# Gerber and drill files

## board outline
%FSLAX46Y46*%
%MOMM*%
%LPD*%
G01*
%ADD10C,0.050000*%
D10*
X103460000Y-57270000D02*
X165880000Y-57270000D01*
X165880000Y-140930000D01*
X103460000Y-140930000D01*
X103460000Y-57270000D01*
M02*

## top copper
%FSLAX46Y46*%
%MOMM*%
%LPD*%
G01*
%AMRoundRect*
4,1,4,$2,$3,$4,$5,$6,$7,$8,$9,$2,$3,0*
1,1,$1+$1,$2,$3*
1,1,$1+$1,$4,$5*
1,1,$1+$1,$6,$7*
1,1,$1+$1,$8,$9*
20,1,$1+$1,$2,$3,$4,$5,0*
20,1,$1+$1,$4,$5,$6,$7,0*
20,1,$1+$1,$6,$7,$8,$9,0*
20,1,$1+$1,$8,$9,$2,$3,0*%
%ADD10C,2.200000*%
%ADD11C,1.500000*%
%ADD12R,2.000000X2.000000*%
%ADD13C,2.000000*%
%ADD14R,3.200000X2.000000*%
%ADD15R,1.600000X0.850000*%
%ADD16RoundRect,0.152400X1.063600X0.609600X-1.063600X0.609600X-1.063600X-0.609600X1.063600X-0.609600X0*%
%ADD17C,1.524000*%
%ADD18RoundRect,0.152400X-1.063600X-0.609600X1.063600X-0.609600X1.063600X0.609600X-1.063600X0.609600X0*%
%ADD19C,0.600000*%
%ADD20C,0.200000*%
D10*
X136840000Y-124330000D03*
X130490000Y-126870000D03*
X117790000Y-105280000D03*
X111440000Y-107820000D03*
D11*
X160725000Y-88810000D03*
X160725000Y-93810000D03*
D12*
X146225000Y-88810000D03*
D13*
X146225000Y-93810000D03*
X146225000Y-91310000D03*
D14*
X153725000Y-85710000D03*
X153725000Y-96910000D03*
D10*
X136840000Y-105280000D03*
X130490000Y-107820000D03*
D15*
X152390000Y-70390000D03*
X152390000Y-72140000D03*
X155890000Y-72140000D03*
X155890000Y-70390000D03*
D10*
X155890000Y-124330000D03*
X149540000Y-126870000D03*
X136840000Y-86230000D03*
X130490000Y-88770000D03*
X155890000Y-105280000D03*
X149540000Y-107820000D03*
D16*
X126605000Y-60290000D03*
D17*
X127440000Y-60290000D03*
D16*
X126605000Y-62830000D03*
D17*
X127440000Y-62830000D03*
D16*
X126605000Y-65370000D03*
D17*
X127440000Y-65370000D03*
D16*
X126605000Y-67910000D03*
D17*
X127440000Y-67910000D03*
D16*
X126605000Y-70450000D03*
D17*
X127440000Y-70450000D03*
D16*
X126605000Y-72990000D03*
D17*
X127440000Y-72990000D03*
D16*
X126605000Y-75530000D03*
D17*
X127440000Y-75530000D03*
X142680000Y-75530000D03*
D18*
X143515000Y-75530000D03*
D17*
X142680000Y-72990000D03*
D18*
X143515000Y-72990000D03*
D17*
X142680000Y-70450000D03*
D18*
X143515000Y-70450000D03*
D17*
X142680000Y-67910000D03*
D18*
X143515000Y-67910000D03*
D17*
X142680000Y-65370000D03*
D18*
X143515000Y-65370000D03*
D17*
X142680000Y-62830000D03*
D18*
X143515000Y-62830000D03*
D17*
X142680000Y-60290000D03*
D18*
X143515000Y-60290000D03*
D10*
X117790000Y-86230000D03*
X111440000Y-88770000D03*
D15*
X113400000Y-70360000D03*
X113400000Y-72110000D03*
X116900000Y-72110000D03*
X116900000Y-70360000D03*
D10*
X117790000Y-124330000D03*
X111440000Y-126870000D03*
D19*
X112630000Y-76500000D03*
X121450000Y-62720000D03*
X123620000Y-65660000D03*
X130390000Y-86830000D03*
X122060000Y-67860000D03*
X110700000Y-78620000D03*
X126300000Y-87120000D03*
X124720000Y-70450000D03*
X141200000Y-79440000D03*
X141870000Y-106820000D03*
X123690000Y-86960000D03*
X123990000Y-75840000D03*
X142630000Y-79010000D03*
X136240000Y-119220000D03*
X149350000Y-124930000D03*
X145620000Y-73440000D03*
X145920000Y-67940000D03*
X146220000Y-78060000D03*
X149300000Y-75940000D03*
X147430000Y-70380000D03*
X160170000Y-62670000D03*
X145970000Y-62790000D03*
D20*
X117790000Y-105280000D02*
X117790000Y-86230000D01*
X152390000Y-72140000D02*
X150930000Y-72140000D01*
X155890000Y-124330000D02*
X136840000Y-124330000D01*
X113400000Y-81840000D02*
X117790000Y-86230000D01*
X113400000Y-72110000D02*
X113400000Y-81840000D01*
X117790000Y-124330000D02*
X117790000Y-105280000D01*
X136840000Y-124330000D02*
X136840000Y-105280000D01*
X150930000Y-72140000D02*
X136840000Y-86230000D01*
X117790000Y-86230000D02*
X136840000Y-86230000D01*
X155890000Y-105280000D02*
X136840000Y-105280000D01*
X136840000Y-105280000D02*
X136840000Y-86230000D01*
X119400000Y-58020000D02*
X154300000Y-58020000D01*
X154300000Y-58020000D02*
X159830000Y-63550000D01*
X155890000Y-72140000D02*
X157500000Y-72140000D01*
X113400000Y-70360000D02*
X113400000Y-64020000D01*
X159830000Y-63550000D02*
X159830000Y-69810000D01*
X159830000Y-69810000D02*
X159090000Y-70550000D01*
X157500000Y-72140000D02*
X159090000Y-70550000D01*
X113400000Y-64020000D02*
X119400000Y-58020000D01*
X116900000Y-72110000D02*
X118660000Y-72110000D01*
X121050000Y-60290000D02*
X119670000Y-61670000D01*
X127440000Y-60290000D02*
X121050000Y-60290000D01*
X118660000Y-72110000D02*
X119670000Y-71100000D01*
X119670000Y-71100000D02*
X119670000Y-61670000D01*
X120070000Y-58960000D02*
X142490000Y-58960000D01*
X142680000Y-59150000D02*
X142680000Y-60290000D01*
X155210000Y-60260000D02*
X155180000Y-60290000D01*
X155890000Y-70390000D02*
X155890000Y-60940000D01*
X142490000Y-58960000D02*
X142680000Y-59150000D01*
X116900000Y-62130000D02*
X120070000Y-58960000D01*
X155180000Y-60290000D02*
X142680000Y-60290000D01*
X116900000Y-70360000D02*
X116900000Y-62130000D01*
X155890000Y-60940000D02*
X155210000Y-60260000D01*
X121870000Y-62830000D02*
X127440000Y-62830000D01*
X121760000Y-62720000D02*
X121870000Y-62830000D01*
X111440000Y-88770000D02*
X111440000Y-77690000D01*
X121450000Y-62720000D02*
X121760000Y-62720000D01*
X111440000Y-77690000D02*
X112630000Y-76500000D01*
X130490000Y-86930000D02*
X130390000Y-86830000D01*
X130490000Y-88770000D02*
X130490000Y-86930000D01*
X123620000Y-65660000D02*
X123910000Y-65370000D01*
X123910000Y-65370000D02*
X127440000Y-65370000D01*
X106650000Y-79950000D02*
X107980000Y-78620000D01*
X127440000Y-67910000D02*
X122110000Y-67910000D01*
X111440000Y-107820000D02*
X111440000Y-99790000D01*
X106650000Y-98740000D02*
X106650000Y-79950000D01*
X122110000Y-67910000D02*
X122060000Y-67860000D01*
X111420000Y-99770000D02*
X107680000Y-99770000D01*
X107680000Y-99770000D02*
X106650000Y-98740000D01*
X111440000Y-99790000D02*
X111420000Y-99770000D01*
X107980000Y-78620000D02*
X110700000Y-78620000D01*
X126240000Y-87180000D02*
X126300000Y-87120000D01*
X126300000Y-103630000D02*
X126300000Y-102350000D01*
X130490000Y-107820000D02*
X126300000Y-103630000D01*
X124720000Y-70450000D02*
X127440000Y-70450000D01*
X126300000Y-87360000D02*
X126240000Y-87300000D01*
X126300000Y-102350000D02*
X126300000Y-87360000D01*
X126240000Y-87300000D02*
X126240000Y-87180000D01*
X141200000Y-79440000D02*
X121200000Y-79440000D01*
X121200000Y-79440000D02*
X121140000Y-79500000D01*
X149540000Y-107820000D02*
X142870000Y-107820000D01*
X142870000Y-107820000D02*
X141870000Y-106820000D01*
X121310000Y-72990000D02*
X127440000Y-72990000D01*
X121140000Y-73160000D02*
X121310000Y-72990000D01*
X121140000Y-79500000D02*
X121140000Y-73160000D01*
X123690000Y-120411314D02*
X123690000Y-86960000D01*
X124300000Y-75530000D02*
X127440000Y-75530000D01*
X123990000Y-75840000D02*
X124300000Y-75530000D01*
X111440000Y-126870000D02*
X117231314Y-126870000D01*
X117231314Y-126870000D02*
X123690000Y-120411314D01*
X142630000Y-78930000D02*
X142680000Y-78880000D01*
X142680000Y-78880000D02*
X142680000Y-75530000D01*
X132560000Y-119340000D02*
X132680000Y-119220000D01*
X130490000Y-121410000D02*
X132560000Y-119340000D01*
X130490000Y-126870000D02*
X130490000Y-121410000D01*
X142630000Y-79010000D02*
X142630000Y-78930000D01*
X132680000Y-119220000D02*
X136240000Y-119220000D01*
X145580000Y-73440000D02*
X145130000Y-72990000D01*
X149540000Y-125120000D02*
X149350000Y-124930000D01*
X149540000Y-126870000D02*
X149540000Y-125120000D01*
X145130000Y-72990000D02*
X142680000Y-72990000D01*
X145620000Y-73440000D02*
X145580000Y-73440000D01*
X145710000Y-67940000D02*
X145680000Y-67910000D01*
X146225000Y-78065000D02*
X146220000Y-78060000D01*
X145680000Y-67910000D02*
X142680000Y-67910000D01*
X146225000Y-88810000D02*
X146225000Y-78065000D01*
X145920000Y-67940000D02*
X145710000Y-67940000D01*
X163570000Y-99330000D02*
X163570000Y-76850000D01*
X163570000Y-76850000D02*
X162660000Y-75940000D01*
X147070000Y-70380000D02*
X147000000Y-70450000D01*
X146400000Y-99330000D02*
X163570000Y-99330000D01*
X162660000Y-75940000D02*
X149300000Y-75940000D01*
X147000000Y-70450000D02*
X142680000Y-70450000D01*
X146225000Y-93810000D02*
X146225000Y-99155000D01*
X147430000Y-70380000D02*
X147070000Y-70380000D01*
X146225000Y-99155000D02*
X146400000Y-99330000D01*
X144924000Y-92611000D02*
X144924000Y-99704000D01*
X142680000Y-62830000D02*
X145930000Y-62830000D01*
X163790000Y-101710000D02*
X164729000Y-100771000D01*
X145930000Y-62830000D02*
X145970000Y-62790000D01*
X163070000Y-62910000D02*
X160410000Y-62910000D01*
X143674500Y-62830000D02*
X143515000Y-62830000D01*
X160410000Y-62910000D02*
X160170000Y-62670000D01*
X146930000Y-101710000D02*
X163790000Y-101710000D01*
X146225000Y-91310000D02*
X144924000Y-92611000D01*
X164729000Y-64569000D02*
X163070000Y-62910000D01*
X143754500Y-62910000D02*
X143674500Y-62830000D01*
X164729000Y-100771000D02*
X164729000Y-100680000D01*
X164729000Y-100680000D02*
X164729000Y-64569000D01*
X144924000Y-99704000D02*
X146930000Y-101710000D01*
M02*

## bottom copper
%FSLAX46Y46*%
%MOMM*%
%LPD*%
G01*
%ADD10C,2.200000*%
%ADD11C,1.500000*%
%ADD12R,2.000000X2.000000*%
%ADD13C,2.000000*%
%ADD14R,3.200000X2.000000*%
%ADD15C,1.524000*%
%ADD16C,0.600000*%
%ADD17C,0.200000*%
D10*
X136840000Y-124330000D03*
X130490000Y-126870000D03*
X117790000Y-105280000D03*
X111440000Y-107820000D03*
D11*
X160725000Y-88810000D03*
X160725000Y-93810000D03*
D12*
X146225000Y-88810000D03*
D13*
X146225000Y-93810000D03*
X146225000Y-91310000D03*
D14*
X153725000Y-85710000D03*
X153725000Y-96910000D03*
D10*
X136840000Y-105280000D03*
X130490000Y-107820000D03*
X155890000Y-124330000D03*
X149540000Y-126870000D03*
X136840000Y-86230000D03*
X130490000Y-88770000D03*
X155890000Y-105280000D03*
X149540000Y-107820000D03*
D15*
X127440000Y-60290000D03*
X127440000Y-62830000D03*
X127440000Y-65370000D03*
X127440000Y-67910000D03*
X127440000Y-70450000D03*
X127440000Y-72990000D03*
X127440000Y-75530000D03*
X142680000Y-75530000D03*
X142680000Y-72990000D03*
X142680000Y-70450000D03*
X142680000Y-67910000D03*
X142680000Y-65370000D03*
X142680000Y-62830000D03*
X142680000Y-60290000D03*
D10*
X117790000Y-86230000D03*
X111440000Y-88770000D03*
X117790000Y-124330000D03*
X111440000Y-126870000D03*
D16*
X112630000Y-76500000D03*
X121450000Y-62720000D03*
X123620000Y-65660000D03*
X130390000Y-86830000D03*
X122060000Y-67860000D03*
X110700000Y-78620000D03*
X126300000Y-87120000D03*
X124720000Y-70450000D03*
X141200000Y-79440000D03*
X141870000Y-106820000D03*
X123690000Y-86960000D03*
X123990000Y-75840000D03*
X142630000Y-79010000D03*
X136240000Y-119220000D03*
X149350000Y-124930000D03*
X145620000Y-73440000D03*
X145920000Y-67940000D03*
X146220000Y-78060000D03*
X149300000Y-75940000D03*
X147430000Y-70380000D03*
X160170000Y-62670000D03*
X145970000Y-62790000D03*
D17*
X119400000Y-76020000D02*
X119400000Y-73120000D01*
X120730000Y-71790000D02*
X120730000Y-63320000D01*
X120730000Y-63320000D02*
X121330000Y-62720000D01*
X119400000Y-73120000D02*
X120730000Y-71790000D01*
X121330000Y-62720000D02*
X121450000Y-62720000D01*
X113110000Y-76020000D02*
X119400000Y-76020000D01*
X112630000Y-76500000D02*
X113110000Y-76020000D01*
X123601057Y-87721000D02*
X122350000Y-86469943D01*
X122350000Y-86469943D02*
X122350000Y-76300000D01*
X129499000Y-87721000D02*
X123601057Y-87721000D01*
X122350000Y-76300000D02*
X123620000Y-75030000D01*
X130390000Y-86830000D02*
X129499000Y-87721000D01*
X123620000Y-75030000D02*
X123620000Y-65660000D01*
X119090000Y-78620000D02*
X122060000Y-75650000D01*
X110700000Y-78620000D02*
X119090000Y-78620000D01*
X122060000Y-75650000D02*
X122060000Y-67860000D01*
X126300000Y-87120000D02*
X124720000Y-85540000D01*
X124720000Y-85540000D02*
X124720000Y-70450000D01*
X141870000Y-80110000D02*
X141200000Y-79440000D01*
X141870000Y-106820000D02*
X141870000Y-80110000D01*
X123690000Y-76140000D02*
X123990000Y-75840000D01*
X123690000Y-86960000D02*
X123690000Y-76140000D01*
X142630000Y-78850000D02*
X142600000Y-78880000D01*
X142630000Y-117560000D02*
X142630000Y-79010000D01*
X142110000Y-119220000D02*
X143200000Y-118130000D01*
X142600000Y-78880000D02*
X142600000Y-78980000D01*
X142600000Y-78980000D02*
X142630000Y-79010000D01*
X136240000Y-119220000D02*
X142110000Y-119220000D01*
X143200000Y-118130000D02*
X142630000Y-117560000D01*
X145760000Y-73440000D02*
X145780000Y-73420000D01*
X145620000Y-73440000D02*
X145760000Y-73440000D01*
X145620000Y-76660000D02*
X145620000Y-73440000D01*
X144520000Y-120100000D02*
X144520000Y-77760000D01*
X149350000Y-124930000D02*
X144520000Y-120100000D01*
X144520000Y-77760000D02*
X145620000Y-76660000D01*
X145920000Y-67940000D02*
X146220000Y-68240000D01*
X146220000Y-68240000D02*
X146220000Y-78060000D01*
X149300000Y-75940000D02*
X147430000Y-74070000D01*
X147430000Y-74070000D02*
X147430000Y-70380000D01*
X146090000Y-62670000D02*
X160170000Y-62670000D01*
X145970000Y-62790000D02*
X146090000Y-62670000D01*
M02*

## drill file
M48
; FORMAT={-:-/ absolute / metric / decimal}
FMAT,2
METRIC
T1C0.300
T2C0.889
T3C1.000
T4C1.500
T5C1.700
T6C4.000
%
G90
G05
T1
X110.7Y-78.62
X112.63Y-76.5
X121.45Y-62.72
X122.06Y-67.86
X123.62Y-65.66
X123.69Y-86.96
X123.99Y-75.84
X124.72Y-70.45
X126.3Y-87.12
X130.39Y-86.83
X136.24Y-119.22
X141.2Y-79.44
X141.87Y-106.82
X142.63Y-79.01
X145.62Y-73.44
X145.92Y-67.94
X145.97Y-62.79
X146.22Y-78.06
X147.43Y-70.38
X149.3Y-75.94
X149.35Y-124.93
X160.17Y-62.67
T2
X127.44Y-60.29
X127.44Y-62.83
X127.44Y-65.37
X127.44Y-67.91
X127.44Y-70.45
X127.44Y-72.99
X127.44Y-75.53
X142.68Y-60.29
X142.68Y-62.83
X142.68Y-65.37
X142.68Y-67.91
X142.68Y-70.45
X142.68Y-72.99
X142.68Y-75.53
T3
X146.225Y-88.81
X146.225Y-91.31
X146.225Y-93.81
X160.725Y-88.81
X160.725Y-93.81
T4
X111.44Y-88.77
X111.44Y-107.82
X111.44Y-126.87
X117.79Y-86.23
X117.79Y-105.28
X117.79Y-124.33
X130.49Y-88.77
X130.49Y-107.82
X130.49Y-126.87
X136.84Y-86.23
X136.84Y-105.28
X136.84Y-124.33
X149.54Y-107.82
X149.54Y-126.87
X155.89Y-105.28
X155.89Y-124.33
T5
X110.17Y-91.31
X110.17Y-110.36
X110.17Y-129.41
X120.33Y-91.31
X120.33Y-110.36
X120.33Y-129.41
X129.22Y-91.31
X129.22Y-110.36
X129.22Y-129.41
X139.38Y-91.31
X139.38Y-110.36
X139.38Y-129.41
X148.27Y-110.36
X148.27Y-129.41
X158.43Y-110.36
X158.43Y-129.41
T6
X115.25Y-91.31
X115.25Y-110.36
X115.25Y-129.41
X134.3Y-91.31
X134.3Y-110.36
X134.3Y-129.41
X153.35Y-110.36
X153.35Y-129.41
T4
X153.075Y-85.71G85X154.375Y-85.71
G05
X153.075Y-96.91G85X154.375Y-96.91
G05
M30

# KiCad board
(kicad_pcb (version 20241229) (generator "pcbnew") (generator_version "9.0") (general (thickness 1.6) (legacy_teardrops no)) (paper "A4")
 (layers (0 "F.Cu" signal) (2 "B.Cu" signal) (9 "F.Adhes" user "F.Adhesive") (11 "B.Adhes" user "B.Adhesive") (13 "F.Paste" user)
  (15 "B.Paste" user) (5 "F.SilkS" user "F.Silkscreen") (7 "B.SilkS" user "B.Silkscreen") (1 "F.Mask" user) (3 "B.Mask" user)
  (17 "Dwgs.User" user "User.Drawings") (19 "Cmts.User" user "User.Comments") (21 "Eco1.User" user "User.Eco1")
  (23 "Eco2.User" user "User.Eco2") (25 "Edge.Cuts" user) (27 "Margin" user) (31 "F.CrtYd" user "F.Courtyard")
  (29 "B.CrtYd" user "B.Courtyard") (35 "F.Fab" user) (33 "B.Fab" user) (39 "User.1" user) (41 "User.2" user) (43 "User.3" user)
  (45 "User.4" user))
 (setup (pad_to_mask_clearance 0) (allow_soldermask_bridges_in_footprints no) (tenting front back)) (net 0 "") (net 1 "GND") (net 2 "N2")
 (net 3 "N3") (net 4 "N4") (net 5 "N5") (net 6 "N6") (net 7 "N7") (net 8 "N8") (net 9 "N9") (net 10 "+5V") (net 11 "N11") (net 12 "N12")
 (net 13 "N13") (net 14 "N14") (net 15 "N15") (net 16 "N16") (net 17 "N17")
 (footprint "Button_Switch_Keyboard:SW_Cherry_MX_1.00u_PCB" (layer "F.Cu") (at 136.84 124.33)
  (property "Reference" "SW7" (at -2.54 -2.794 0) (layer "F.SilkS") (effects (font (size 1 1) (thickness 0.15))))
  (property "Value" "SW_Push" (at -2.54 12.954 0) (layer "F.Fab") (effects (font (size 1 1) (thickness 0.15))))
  (pad "" np_thru_hole circle (at -7.62 5.08) (size 1.7 1.7) (drill 1.7) (layers "*.Cu" "*.Mask"))
  (pad "" np_thru_hole circle (at -2.54 5.08) (size 4 4) (drill 4) (layers "*.Cu" "*.Mask"))
  (pad "" np_thru_hole circle (at 2.54 5.08) (size 1.7 1.7) (drill 1.7) (layers "*.Cu" "*.Mask"))
  (pad "1" thru_hole circle (at 0 0) (size 2.2 2.2) (drill 1.5) (layers "*.Cu" "*.Mask") (remove_unused_layers no) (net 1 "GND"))
  (pad "2" thru_hole circle (at -6.35 2.54) (size 2.2 2.2) (drill 1.5) (layers "*.Cu" "*.Mask") (remove_unused_layers no) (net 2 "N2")))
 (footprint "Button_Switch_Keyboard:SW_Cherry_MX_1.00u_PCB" (layer "F.Cu") (at 117.79 105.28)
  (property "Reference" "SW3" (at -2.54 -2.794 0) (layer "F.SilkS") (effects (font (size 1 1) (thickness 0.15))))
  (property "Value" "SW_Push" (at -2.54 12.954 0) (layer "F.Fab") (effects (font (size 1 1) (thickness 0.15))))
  (pad "" np_thru_hole circle (at -7.62 5.08) (size 1.7 1.7) (drill 1.7) (layers "*.Cu" "*.Mask"))
  (pad "" np_thru_hole circle (at -2.54 5.08) (size 4 4) (drill 4) (layers "*.Cu" "*.Mask"))
  (pad "" np_thru_hole circle (at 2.54 5.08) (size 1.7 1.7) (drill 1.7) (layers "*.Cu" "*.Mask"))
  (pad "1" thru_hole circle (at 0 0) (size 2.2 2.2) (drill 1.5) (layers "*.Cu" "*.Mask") (remove_unused_layers no) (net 1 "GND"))
  (pad "2" thru_hole circle (at -6.35 2.54) (size 2.2 2.2) (drill 1.5) (layers "*.Cu" "*.Mask") (remove_unused_layers no) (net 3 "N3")))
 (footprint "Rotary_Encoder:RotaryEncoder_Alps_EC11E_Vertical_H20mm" (layer "F.Cu") (at 146.225 88.81)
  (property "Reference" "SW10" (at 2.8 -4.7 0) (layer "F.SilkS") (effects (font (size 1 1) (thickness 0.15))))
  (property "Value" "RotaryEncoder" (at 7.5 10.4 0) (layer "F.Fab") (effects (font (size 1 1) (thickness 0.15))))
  (pad "" thru_hole circle (at 14.5 0) (size 1.5 1.5) (drill 1) (layers "*.Cu" "*.Mask") (remove_unused_layers no))
  (pad "" thru_hole circle (at 14.5 5) (size 1.5 1.5) (drill 1) (layers "*.Cu" "*.Mask") (remove_unused_layers no))
  (pad "A" thru_hole rect (at 0 0) (size 2 2) (drill 1) (layers "*.Cu" "*.Mask") (remove_unused_layers no) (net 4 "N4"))
  (pad "B" thru_hole circle (at 0 5) (size 2 2) (drill 1) (layers "*.Cu" "*.Mask") (remove_unused_layers no) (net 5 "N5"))
  (pad "C" thru_hole circle (at 0 2.5) (size 2 2) (drill 1) (layers "*.Cu" "*.Mask") (remove_unused_layers no) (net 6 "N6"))
  (pad "MP" thru_hole rect (at 7.5 -3.1) (size 3.2 2) (drill oval 2.8 1.5) (layers "*.Cu" "*.Mask") (remove_unused_layers no))
  (pad "MP" thru_hole rect (at 7.5 8.1) (size 3.2 2) (drill oval 2.8 1.5) (layers "*.Cu" "*.Mask") (remove_unused_layers no)))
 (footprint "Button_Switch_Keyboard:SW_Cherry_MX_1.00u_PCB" (layer "F.Cu") (at 136.84 105.28)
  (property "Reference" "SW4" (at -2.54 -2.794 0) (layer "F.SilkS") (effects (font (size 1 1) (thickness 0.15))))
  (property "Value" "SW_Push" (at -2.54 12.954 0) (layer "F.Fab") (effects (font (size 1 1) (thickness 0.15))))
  (pad "" np_thru_hole circle (at -7.62 5.08) (size 1.7 1.7) (drill 1.7) (layers "*.Cu" "*.Mask"))
  (pad "" np_thru_hole circle (at -2.54 5.08) (size 4 4) (drill 4) (layers "*.Cu" "*.Mask"))
  (pad "" np_thru_hole circle (at 2.54 5.08) (size 1.7 1.7) (drill 1.7) (layers "*.Cu" "*.Mask"))
  (pad "1" thru_hole circle (at 0 0) (size 2.2 2.2) (drill 1.5) (layers "*.Cu" "*.Mask") (remove_unused_layers no) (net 1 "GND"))
  (pad "2" thru_hole circle (at -6.35 2.54) (size 2.2 2.2) (drill 1.5) (layers "*.Cu" "*.Mask") (remove_unused_layers no) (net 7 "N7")))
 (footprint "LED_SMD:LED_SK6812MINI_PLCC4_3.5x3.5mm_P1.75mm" (layer "F.Cu") (at 154.14 71.265)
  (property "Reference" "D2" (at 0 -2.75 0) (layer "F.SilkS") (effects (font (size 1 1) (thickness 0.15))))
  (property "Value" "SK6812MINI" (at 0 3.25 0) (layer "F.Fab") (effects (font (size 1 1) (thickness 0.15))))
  (pad "1" smd rect (at -1.75 -0.875) (size 1.6 0.85) (layers "F.Cu" "F.Mask" "F.Paste") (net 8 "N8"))
  (pad "2" smd rect (at -1.75 0.875) (size 1.6 0.85) (layers "F.Cu" "F.Mask" "F.Paste") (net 1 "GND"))
  (pad "3" smd rect (at 1.75 0.875) (size 1.6 0.85) (layers "F.Cu" "F.Mask" "F.Paste") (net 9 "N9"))
  (pad "4" smd rect (at 1.75 -0.875) (size 1.6 0.85) (layers "F.Cu" "F.Mask" "F.Paste") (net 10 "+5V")))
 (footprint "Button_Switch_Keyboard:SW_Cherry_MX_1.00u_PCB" (layer "F.Cu") (at 155.89 124.33)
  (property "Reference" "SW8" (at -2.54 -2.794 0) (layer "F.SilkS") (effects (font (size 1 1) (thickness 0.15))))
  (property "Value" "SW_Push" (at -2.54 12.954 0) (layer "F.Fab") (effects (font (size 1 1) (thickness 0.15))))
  (pad "" np_thru_hole circle (at -7.62 5.08) (size 1.7 1.7) (drill 1.7) (layers "*.Cu" "*.Mask"))
  (pad "" np_thru_hole circle (at -2.54 5.08) (size 4 4) (drill 4) (layers "*.Cu" "*.Mask"))
  (pad "" np_thru_hole circle (at 2.54 5.08) (size 1.7 1.7) (drill 1.7) (layers "*.Cu" "*.Mask"))
  (pad "1" thru_hole circle (at 0 0) (size 2.2 2.2) (drill 1.5) (layers "*.Cu" "*.Mask") (remove_unused_layers no) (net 1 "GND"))
  (pad "2" thru_hole circle (at -6.35 2.54) (size 2.2 2.2) (drill 1.5) (layers "*.Cu" "*.Mask") (remove_unused_layers no) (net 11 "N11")))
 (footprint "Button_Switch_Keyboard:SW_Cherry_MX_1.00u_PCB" (layer "F.Cu") (at 136.84 86.23)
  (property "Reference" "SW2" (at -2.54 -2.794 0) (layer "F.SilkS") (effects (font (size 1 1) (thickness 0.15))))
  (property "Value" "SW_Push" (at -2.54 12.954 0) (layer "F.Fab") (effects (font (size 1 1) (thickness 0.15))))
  (pad "" np_thru_hole circle (at -7.62 5.08) (size 1.7 1.7) (drill 1.7) (layers "*.Cu" "*.Mask"))
  (pad "" np_thru_hole circle (at -2.54 5.08) (size 4 4) (drill 4) (layers "*.Cu" "*.Mask"))
  (pad "" np_thru_hole circle (at 2.54 5.08) (size 1.7 1.7) (drill 1.7) (layers "*.Cu" "*.Mask"))
  (pad "1" thru_hole circle (at 0 0) (size 2.2 2.2) (drill 1.5) (layers "*.Cu" "*.Mask") (remove_unused_layers no) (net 1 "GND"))
  (pad "2" thru_hole circle (at -6.35 2.54) (size 2.2 2.2) (drill 1.5) (layers "*.Cu" "*.Mask") (remove_unused_layers no) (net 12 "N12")))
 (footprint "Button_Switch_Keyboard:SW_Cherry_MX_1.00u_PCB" (layer "F.Cu") (at 155.89 105.28)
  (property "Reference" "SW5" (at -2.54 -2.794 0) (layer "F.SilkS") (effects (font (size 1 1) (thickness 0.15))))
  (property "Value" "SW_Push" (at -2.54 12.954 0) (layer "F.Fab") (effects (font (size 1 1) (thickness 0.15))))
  (pad "" np_thru_hole circle (at -7.62 5.08) (size 1.7 1.7) (drill 1.7) (layers "*.Cu" "*.Mask"))
  (pad "" np_thru_hole circle (at -2.54 5.08) (size 4 4) (drill 4) (layers "*.Cu" "*.Mask"))
  (pad "" np_thru_hole circle (at 2.54 5.08) (size 1.7 1.7) (drill 1.7) (layers "*.Cu" "*.Mask"))
  (pad "1" thru_hole circle (at 0 0) (size 2.2 2.2) (drill 1.5) (layers "*.Cu" "*.Mask") (remove_unused_layers no) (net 1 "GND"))
  (pad "2" thru_hole circle (at -6.35 2.54) (size 2.2 2.2) (drill 1.5) (layers "*.Cu" "*.Mask") (remove_unused_layers no) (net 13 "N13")))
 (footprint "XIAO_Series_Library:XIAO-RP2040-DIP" (layer "F.Cu") (at 135.06 67.91)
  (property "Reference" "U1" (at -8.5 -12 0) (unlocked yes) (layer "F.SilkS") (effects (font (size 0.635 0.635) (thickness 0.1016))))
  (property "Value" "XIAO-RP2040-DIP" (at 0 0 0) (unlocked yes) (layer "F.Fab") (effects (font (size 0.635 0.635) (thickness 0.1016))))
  (pad "1" smd roundrect (at -8.455 -7.62 180) (size 2.432 1.524) (layers "F.Cu" "F.Mask") (roundrect_rratio 0.1) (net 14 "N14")
   (thermal_bridge_angle 45))
  (pad "1" thru_hole circle (at -7.62 -7.62 180) (size 1.524 1.524) (drill 0.889) (layers "*.Cu" "*.Mask") (remove_unused_layers no)
   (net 14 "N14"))
  (pad "2" smd roundrect (at -8.455 -5.08 180) (size 2.432 1.524) (layers "F.Cu" "F.Mask") (roundrect_rratio 0.1) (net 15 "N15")
   (thermal_bridge_angle 45))
  (pad "2" thru_hole circle (at -7.62 -5.08 180) (size 1.524 1.524) (drill 0.889) (layers "*.Cu" "*.Mask") (remove_unused_layers no)
   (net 15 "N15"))
  (pad "3" smd roundrect (at -8.455 -2.54 180) (size 2.432 1.524) (layers "F.Cu" "F.Mask") (roundrect_rratio 0.1) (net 12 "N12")
   (thermal_bridge_angle 45))
  (pad "3" thru_hole circle (at -7.62 -2.54 180) (size 1.524 1.524) (drill 0.889) (layers "*.Cu" "*.Mask") (remove_unused_layers no)
   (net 12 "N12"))
  (pad "4" smd roundrect (at -8.455 0 180) (size 2.432 1.524) (layers "F.Cu" "F.Mask") (roundrect_rratio 0.1) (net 3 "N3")
   (thermal_bridge_angle 45))
  (pad "4" thru_hole circle (at -7.62 0 180) (size 1.524 1.524) (drill 0.889) (layers "*.Cu" "*.Mask") (remove_unused_layers no)
   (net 3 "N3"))
  (pad "5" smd roundrect (at -8.455 2.54 180) (size 2.432 1.524) (layers "F.Cu" "F.Mask") (roundrect_rratio 0.1) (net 7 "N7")
   (thermal_bridge_angle 45))
  (pad "5" thru_hole circle (at -7.62 2.54 180) (size 1.524 1.524) (drill 0.889) (layers "*.Cu" "*.Mask") (remove_unused_layers no)
   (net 7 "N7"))
  (pad "6" smd roundrect (at -8.455 5.08 180) (size 2.432 1.524) (layers "F.Cu" "F.Mask") (roundrect_rratio 0.1) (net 13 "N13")
   (thermal_bridge_angle 45))
  (pad "6" thru_hole circle (at -7.62 5.08 180) (size 1.524 1.524) (drill 0.889) (layers "*.Cu" "*.Mask") (remove_unused_layers no)
   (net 13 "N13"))
  (pad "7" smd roundrect (at -8.455 7.62 180) (size 2.432 1.524) (layers "F.Cu" "F.Mask") (roundrect_rratio 0.1) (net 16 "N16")
   (thermal_bridge_angle 45))
  (pad "7" thru_hole circle (at -7.62 7.62 180) (size 1.524 1.524) (drill 0.889) (layers "*.Cu" "*.Mask") (remove_unused_layers no)
   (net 16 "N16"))
  (pad "8" thru_hole circle (at 7.62 7.62) (size 1.524 1.524) (drill 0.889) (layers "*.Cu" "*.Mask") (remove_unused_layers no) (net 2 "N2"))
  (pad "8" smd roundrect (at 8.455 7.62) (size 2.432 1.524) (layers "F.Cu" "F.Mask") (roundrect_rratio 0.1) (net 2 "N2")
   (thermal_bridge_angle 45))
  (pad "9" thru_hole circle (at 7.62 5.08) (size 1.524 1.524) (drill 0.889) (layers "*.Cu" "*.Mask") (remove_unused_layers no)
   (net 11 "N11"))
  (pad "9" smd roundrect (at 8.455 5.08) (size 2.432 1.524) (layers "F.Cu" "F.Mask") (roundrect_rratio 0.1) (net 11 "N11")
   (thermal_bridge_angle 45))
  (pad "10" thru_hole circle (at 7.62 2.54) (size 1.524 1.524) (drill 0.889) (layers "*.Cu" "*.Mask") (remove_unused_layers no) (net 5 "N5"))
  (pad "10" smd roundrect (at 8.455 2.54) (size 2.432 1.524) (layers "F.Cu" "F.Mask") (roundrect_rratio 0.1) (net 5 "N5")
   (thermal_bridge_angle 45))
  (pad "11" thru_hole circle (at 7.62 0) (size 1.524 1.524) (drill 0.889) (layers "*.Cu" "*.Mask") (remove_unused_layers no) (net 4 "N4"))
  (pad "11" smd roundrect (at 8.455 0) (size 2.432 1.524) (layers "F.Cu" "F.Mask") (roundrect_rratio 0.1) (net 4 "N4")
   (thermal_bridge_angle 45))
  (pad "12" thru_hole circle (at 7.62 -2.54) (size 1.524 1.524) (drill 0.889) (layers "*.Cu" "*.Mask") (remove_unused_layers no)
   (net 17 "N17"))
  (pad "12" smd roundrect (at 8.455 -2.54) (size 2.432 1.524) (layers "F.Cu" "F.Mask") (roundrect_rratio 0.1) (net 17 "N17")
   (thermal_bridge_angle 45))
  (pad "13" thru_hole circle (at 7.62 -5.08) (size 1.524 1.524) (drill 0.889) (layers "*.Cu" "*.Mask") (remove_unused_layers no)
   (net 6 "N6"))
  (pad "13" smd roundrect (at 8.455 -5.08) (size 2.432 1.524) (layers "F.Cu" "F.Mask") (roundrect_rratio 0.1) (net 6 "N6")
   (thermal_bridge_angle 45))
  (pad "14" thru_hole circle (at 7.62 -7.62) (size 1.524 1.524) (drill 0.889) (layers "*.Cu" "*.Mask") (remove_unused_layers no)
   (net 10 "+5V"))
  (pad "14" smd roundrect (at 8.455 -7.62) (size 2.432 1.524) (layers "F.Cu" "F.Mask") (roundrect_rratio 0.1) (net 10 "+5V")
   (thermal_bridge_angle 45)))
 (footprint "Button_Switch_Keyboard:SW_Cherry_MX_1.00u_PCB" (layer "F.Cu") (at 117.79 86.23)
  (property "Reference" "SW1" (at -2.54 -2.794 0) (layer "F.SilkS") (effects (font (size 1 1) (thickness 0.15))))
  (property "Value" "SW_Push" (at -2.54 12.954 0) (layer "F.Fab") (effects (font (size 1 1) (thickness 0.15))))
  (pad "" np_thru_hole circle (at -7.62 5.08) (size 1.7 1.7) (drill 1.7) (layers "*.Cu" "*.Mask"))
  (pad "" np_thru_hole circle (at -2.54 5.08) (size 4 4) (drill 4) (layers "*.Cu" "*.Mask"))
  (pad "" np_thru_hole circle (at 2.54 5.08) (size 1.7 1.7) (drill 1.7) (layers "*.Cu" "*.Mask"))
  (pad "1" thru_hole circle (at 0 0) (size 2.2 2.2) (drill 1.5) (layers "*.Cu" "*.Mask") (remove_unused_layers no) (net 1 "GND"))
  (pad "2" thru_hole circle (at -6.35 2.54) (size 2.2 2.2) (drill 1.5) (layers "*.Cu" "*.Mask") (remove_unused_layers no) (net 15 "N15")))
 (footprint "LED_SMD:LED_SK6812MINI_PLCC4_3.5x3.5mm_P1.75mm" (layer "F.Cu") (at 115.15 71.235)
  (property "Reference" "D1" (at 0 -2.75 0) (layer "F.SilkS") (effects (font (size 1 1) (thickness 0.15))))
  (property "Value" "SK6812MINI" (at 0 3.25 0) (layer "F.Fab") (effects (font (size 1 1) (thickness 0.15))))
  (pad "1" smd rect (at -1.75 -0.875) (size 1.6 0.85) (layers "F.Cu" "F.Mask" "F.Paste") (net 9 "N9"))
  (pad "2" smd rect (at -1.75 0.875) (size 1.6 0.85) (layers "F.Cu" "F.Mask" "F.Paste") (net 1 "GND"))
  (pad "3" smd rect (at 1.75 0.875) (size 1.6 0.85) (layers "F.Cu" "F.Mask" "F.Paste") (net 14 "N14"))
  (pad "4" smd rect (at 1.75 -0.875) (size 1.6 0.85) (layers "F.Cu" "F.Mask" "F.Paste") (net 10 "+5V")))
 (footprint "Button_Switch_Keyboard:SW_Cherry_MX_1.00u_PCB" (layer "F.Cu") (at 117.79 124.33)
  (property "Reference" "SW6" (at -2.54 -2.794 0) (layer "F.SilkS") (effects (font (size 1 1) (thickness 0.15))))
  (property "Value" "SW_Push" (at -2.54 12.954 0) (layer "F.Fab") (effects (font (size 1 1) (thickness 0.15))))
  (pad "" np_thru_hole circle (at -7.62 5.08) (size 1.7 1.7) (drill 1.7) (layers "*.Cu" "*.Mask"))
  (pad "" np_thru_hole circle (at -2.54 5.08) (size 4 4) (drill 4) (layers "*.Cu" "*.Mask"))
  (pad "" np_thru_hole circle (at 2.54 5.08) (size 1.7 1.7) (drill 1.7) (layers "*.Cu" "*.Mask"))
  (pad "1" thru_hole circle (at 0 0) (size 2.2 2.2) (drill 1.5) (layers "*.Cu" "*.Mask") (remove_unused_layers no) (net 1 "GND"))
  (pad "2" thru_hole circle (at -6.35 2.54) (size 2.2 2.2) (drill 1.5) (layers "*.Cu" "*.Mask") (remove_unused_layers no) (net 16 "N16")))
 (gr_rect (start 103.46 57.27) (end 165.88 140.93) (stroke (width 0.05) (type default)) (fill no) (layer "Edge.Cuts"))
 (segment (start 117.79 105.28) (end 117.79 86.23) (width 0.2) (layer "F.Cu") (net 1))
 (segment (start 152.39 72.14) (end 150.93 72.14) (width 0.2) (layer "F.Cu") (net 1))
 (segment (start 155.89 124.33) (end 136.84 124.33) (width 0.2) (layer "F.Cu") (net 1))
 (segment (start 113.4 81.84) (end 117.79 86.23) (width 0.2) (layer "F.Cu") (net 1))
 (segment (start 113.4 72.11) (end 113.4 81.84) (width 0.2) (layer "F.Cu") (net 1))
 (segment (start 117.79 124.33) (end 117.79 105.28) (width 0.2) (layer "F.Cu") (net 1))
 (segment (start 136.84 124.33) (end 136.84 105.28) (width 0.2) (layer "F.Cu") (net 1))
 (segment (start 150.93 72.14) (end 136.84 86.23) (width 0.2) (layer "F.Cu") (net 1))
 (segment (start 117.79 86.23) (end 136.84 86.23) (width 0.2) (layer "F.Cu") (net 1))
 (segment (start 155.89 105.28) (end 136.84 105.28) (width 0.2) (layer "F.Cu") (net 1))
 (segment (start 136.84 105.28) (end 136.84 86.23) (width 0.2) (layer "F.Cu") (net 1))
 (segment (start 119.4 58.02) (end 154.3 58.02) (width 0.2) (layer "F.Cu") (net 9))
 (segment (start 154.3 58.02) (end 159.83 63.55) (width 0.2) (layer "F.Cu") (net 9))
 (segment (start 155.89 72.14) (end 157.5 72.14) (width 0.2) (layer "F.Cu") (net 9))
 (segment (start 113.4 70.36) (end 113.4 64.02) (width 0.2) (layer "F.Cu") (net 9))
 (segment (start 159.83 63.55) (end 159.83 69.81) (width 0.2) (layer "F.Cu") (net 9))
 (segment (start 159.83 69.81) (end 159.09 70.55) (width 0.2) (layer "F.Cu") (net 9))
 (segment (start 157.5 72.14) (end 159.09 70.55) (width 0.2) (layer "F.Cu") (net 9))
 (segment (start 113.4 64.02) (end 119.4 58.02) (width 0.2) (layer "F.Cu") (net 9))
 (segment (start 116.9 72.11) (end 118.66 72.11) (width 0.2) (layer "F.Cu") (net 14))
 (segment (start 121.05 60.29) (end 119.67 61.67) (width 0.2) (layer "F.Cu") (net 14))
 (segment (start 127.44 60.29) (end 121.05 60.29) (width 0.2) (layer "F.Cu") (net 14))
 (segment (start 118.66 72.11) (end 119.67 71.1) (width 0.2) (layer "F.Cu") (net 14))
 (segment (start 119.67 71.1) (end 119.67 61.67) (width 0.2) (layer "F.Cu") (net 14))
 (segment (start 120.07 58.96) (end 142.49 58.96) (width 0.2) (layer "F.Cu") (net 10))
 (segment (start 142.68 59.15) (end 142.68 60.29) (width 0.2) (layer "F.Cu") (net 10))
 (segment (start 155.21 60.26) (end 155.18 60.29) (width 0.2) (layer "F.Cu") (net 10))
 (segment (start 155.89 70.39) (end 155.89 60.94) (width 0.2) (layer "F.Cu") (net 10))
 (segment (start 142.49 58.96) (end 142.68 59.15) (width 0.2) (layer "F.Cu") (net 10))
 (segment (start 116.9 62.13) (end 120.07 58.96) (width 0.2) (layer "F.Cu") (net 10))
 (segment (start 155.18 60.29) (end 142.68 60.29) (width 0.2) (layer "F.Cu") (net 10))
 (segment (start 116.9 70.36) (end 116.9 62.13) (width 0.2) (layer "F.Cu") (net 10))
 (segment (start 155.89 60.94) (end 155.21 60.26) (width 0.2) (layer "F.Cu") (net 10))
 (segment (start 121.87 62.83) (end 127.44 62.83) (width 0.2) (layer "F.Cu") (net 15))
 (segment (start 121.76 62.72) (end 121.87 62.83) (width 0.2) (layer "F.Cu") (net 15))
 (segment (start 111.44 88.77) (end 111.44 77.69) (width 0.2) (layer "F.Cu") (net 15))
 (segment (start 121.45 62.72) (end 121.76 62.72) (width 0.2) (layer "F.Cu") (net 15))
 (segment (start 111.44 77.69) (end 112.63 76.5) (width 0.2) (layer "F.Cu") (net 15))
 (via (at 112.63 76.5) (size 0.6) (drill 0.3) (layers "F.Cu" "B.Cu") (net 15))
 (via (at 121.45 62.72) (size 0.6) (drill 0.3) (layers "F.Cu" "B.Cu") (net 15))
 (segment (start 119.4 76.02) (end 119.4 73.12) (width 0.2) (layer "B.Cu") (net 15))
 (segment (start 120.73 71.79) (end 120.73 63.32) (width 0.2) (layer "B.Cu") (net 15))
 (segment (start 120.73 63.32) (end 121.33 62.72) (width 0.2) (layer "B.Cu") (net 15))
 (segment (start 119.4 73.12) (end 120.73 71.79) (width 0.2) (layer "B.Cu") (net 15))
 (segment (start 121.33 62.72) (end 121.45 62.72) (width 0.2) (layer "B.Cu") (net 15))
 (segment (start 113.11 76.02) (end 119.4 76.02) (width 0.2) (layer "B.Cu") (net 15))
 (segment (start 112.63 76.5) (end 113.11 76.02) (width 0.2) (layer "B.Cu") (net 15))
 (segment (start 130.49 86.93) (end 130.39 86.83) (width 0.2) (layer "F.Cu") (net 12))
 (segment (start 130.49 88.77) (end 130.49 86.93) (width 0.2) (layer "F.Cu") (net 12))
 (segment (start 123.62 65.66) (end 123.91 65.37) (width 0.2) (layer "F.Cu") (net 12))
 (segment (start 123.91 65.37) (end 127.44 65.37) (width 0.2) (layer "F.Cu") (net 12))
 (via (at 123.62 65.66) (size 0.6) (drill 0.3) (layers "F.Cu" "B.Cu") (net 12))
 (via (at 130.39 86.83) (size 0.6) (drill 0.3) (layers "F.Cu" "B.Cu") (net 12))
 (segment (start 123.601057 87.721) (end 122.35 86.469943) (width 0.2) (layer "B.Cu") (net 12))
 (segment (start 122.35 86.469943) (end 122.35 76.3) (width 0.2) (layer "B.Cu") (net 12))
 (segment (start 129.499 87.721) (end 123.601057 87.721) (width 0.2) (layer "B.Cu") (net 12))
 (segment (start 122.35 76.3) (end 123.62 75.03) (width 0.2) (layer "B.Cu") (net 12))
 (segment (start 130.39 86.83) (end 129.499 87.721) (width 0.2) (layer "B.Cu") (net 12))
 (segment (start 123.62 75.03) (end 123.62 65.66) (width 0.2) (layer "B.Cu") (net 12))
 (segment (start 106.65 79.95) (end 107.98 78.62) (width 0.2) (layer "F.Cu") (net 3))
 (segment (start 127.44 67.91) (end 122.11 67.91) (width 0.2) (layer "F.Cu") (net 3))
 (segment (start 111.44 107.82) (end 111.44 99.79) (width 0.2) (layer "F.Cu") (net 3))
 (segment (start 106.65 98.74) (end 106.65 79.95) (width 0.2) (layer "F.Cu") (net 3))
 (segment (start 122.11 67.91) (end 122.06 67.86) (width 0.2) (layer "F.Cu") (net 3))
 (segment (start 111.42 99.77) (end 107.68 99.77) (width 0.2) (layer "F.Cu") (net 3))
 (segment (start 107.68 99.77) (end 106.65 98.74) (width 0.2) (layer "F.Cu") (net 3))
 (segment (start 111.44 99.79) (end 111.42 99.77) (width 0.2) (layer "F.Cu") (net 3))
 (segment (start 107.98 78.62) (end 110.7 78.62) (width 0.2) (layer "F.Cu") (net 3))
 (via (at 122.06 67.86) (size 0.6) (drill 0.3) (layers "F.Cu" "B.Cu") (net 3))
 (via (at 110.7 78.62) (size 0.6) (drill 0.3) (layers "F.Cu" "B.Cu") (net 3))
 (segment (start 119.09 78.62) (end 122.06 75.65) (width 0.2) (layer "B.Cu") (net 3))
 (segment (start 110.7 78.62) (end 119.09 78.62) (width 0.2) (layer "B.Cu") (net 3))
 (segment (start 122.06 75.65) (end 122.06 67.86) (width 0.2) (layer "B.Cu") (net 3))
 (segment (start 126.24 87.18) (end 126.3 87.12) (width 0.2) (layer "F.Cu") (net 7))
 (segment (start 126.3 103.63) (end 126.3 102.35) (width 0.2) (layer "F.Cu") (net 7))
 (segment (start 130.49 107.82) (end 126.3 103.63) (width 0.2) (layer "F.Cu") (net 7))
 (segment (start 124.72 70.45) (end 127.44 70.45) (width 0.2) (layer "F.Cu") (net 7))
 (segment (start 126.3 87.36) (end 126.24 87.3) (width 0.2) (layer "F.Cu") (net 7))
 (segment (start 126.3 102.35) (end 126.3 87.36) (width 0.2) (layer "F.Cu") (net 7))
 (segment (start 126.24 87.3) (end 126.24 87.18) (width 0.2) (layer "F.Cu") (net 7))
 (via (at 126.3 87.12) (size 0.6) (drill 0.3) (layers "F.Cu" "B.Cu") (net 7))
 (via (at 124.72 70.45) (size 0.6) (drill 0.3) (layers "F.Cu" "B.Cu") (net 7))
 (segment (start 126.3 87.12) (end 124.72 85.54) (width 0.2) (layer "B.Cu") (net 7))
 (segment (start 124.72 85.54) (end 124.72 70.45) (width 0.2) (layer "B.Cu") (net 7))
 (segment (start 141.2 79.44) (end 121.2 79.44) (width 0.2) (layer "F.Cu") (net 13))
 (segment (start 121.2 79.44) (end 121.14 79.5) (width 0.2) (layer "F.Cu") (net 13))
 (segment (start 149.54 107.82) (end 142.87 107.82) (width 0.2) (layer "F.Cu") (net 13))
 (segment (start 142.87 107.82) (end 141.87 106.82) (width 0.2) (layer "F.Cu") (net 13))
 (segment (start 121.31 72.99) (end 127.44 72.99) (width 0.2) (layer "F.Cu") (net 13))
 (segment (start 121.14 73.16) (end 121.31 72.99) (width 0.2) (layer "F.Cu") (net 13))
 (segment (start 121.14 79.5) (end 121.14 73.16) (width 0.2) (layer "F.Cu") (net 13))
 (via (at 141.2 79.44) (size 0.6) (drill 0.3) (layers "F.Cu" "B.Cu") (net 13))
 (via (at 141.87 106.82) (size 0.6) (drill 0.3) (layers "F.Cu" "B.Cu") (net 13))
 (segment (start 141.87 80.11) (end 141.2 79.44) (width 0.2) (layer "B.Cu") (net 13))
 (segment (start 141.87 106.82) (end 141.87 80.11) (width 0.2) (layer "B.Cu") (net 13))
 (segment (start 123.69 120.411314) (end 123.69 86.96) (width 0.2) (layer "F.Cu") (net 16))
 (segment (start 124.3 75.53) (end 127.44 75.53) (width 0.2) (layer "F.Cu") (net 16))
 (segment (start 123.99 75.84) (end 124.3 75.53) (width 0.2) (layer "F.Cu") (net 16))
 (segment (start 111.44 126.87) (end 117.231314 126.87) (width 0.2) (layer "F.Cu") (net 16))
 (segment (start 117.231314 126.87) (end 123.69 120.411314) (width 0.2) (layer "F.Cu") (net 16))
 (via (at 123.69 86.96) (size 0.6) (drill 0.3) (layers "F.Cu" "B.Cu") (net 16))
 (via (at 123.99 75.84) (size 0.6) (drill 0.3) (layers "F.Cu" "B.Cu") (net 16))
 (segment (start 123.69 76.14) (end 123.99 75.84) (width 0.2) (layer "B.Cu") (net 16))
 (segment (start 123.69 86.96) (end 123.69 76.14) (width 0.2) (layer "B.Cu") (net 16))
 (segment (start 142.63 78.93) (end 142.68 78.88) (width 0.2) (layer "F.Cu") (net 2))
 (segment (start 142.68 78.88) (end 142.68 75.53) (width 0.2) (layer "F.Cu") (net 2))
 (segment (start 132.56 119.34) (end 132.68 119.22) (width 0.2) (layer "F.Cu") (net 2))
 (segment (start 130.49 121.41) (end 132.56 119.34) (width 0.2) (layer "F.Cu") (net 2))
 (segment (start 130.49 126.87) (end 130.49 121.41) (width 0.2) (layer "F.Cu") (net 2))
 (segment (start 142.63 79.01) (end 142.63 78.93) (width 0.2) (layer "F.Cu") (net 2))
 (segment (start 132.68 119.22) (end 136.24 119.22) (width 0.2) (layer "F.Cu") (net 2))
 (via (at 142.63 79.01) (size 0.6) (drill 0.3) (layers "F.Cu" "B.Cu") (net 2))
 (via (at 136.24 119.22) (size 0.6) (drill 0.3) (layers "F.Cu" "B.Cu") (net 2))
 (segment (start 142.63 78.85) (end 142.6 78.88) (width 0.2) (layer "B.Cu") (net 2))
 (segment (start 142.63 117.56) (end 142.63 79.01) (width 0.2) (layer "B.Cu") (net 2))
 (segment (start 142.11 119.22) (end 143.2 118.13) (width 0.2) (layer "B.Cu") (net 2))
 (segment (start 142.6 78.88) (end 142.6 78.98) (width 0.2) (layer "B.Cu") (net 2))
 (segment (start 142.6 78.98) (end 142.63 79.01) (width 0.2) (layer "B.Cu") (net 2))
 (segment (start 136.24 119.22) (end 142.11 119.22) (width 0.2) (layer "B.Cu") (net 2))
 (segment (start 143.2 118.13) (end 142.63 117.56) (width 0.2) (layer "B.Cu") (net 2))
 (segment (start 145.58 73.44) (end 145.13 72.99) (width 0.2) (layer "F.Cu") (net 11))
 (segment (start 149.54 125.12) (end 149.35 124.93) (width 0.2) (layer "F.Cu") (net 11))
 (segment (start 149.54 126.87) (end 149.54 125.12) (width 0.2) (layer "F.Cu") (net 11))
 (segment (start 145.13 72.99) (end 142.68 72.99) (width 0.2) (layer "F.Cu") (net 11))
 (segment (start 145.62 73.44) (end 145.58 73.44) (width 0.2) (layer "F.Cu") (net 11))
 (via (at 149.35 124.93) (size 0.6) (drill 0.3) (layers "F.Cu" "B.Cu") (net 11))
 (via (at 145.62 73.44) (size 0.6) (drill 0.3) (layers "F.Cu" "B.Cu") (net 11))
 (segment (start 145.76 73.44) (end 145.78 73.42) (width 0.2) (layer "B.Cu") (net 11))
 (segment (start 145.62 73.44) (end 145.76 73.44) (width 0.2) (layer "B.Cu") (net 11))
 (segment (start 145.62 76.66) (end 145.62 73.44) (width 0.2) (layer "B.Cu") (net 11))
 (segment (start 144.52 120.1) (end 144.52 77.76) (width 0.2) (layer "B.Cu") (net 11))
 (segment (start 149.35 124.93) (end 144.52 120.1) (width 0.2) (layer "B.Cu") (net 11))
 (segment (start 144.52 77.76) (end 145.62 76.66) (width 0.2) (layer "B.Cu") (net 11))
 (segment (start 145.71 67.94) (end 145.68 67.91) (width 0.2) (layer "F.Cu") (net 4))
 (segment (start 146.225 78.065) (end 146.22 78.06) (width 0.2) (layer "F.Cu") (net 4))
 (segment (start 145.68 67.91) (end 142.68 67.91) (width 0.2) (layer "F.Cu") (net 4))
 (segment (start 146.225 88.81) (end 146.225 78.065) (width 0.2) (layer "F.Cu") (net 4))
 (segment (start 145.92 67.94) (end 145.71 67.94) (width 0.2) (layer "F.Cu") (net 4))
 (via (at 145.92 67.94) (size 0.6) (drill 0.3) (layers "F.Cu" "B.Cu") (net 4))
 (via (at 146.22 78.06) (size 0.6) (drill 0.3) (layers "F.Cu" "B.Cu") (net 4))
 (segment (start 145.92 67.94) (end 146.22 68.24) (width 0.2) (layer "B.Cu") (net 4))
 (segment (start 146.22 68.24) (end 146.22 78.06) (width 0.2) (layer "B.Cu") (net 4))
 (segment (start 163.57 99.33) (end 163.57 76.85) (width 0.2) (layer "F.Cu") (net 5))
 (segment (start 163.57 76.85) (end 162.66 75.94) (width 0.2) (layer "F.Cu") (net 5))
 (segment (start 147.07 70.38) (end 147 70.45) (width 0.2) (layer "F.Cu") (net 5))
 (segment (start 146.4 99.33) (end 163.57 99.33) (width 0.2) (layer "F.Cu") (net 5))
 (segment (start 162.66 75.94) (end 149.3 75.94) (width 0.2) (layer "F.Cu") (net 5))
 (segment (start 147 70.45) (end 142.68 70.45) (width 0.2) (layer "F.Cu") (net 5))
 (segment (start 146.225 93.81) (end 146.225 99.155) (width 0.2) (layer "F.Cu") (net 5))
 (segment (start 147.43 70.38) (end 147.07 70.38) (width 0.2) (layer "F.Cu") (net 5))
 (segment (start 146.225 99.155) (end 146.4 99.33) (width 0.2) (layer "F.Cu") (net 5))
 (via (at 149.3 75.94) (size 0.6) (drill 0.3) (layers "F.Cu" "B.Cu") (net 5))
 (via (at 147.43 70.38) (size 0.6) (drill 0.3) (layers "F.Cu" "B.Cu") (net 5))
 (segment (start 149.3 75.94) (end 147.43 74.07) (width 0.2) (layer "B.Cu") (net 5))
 (segment (start 147.43 74.07) (end 147.43 70.38) (width 0.2) (layer "B.Cu") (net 5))
 (segment (start 144.924 92.611) (end 144.924 99.704) (width 0.2) (layer "F.Cu") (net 6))
 (segment (start 142.68 62.83) (end 145.93 62.83) (width 0.2) (layer "F.Cu") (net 6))
 (segment (start 163.79 101.71) (end 164.729 100.771) (width 0.2) (layer "F.Cu") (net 6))
 (segment (start 145.93 62.83) (end 145.97 62.79) (width 0.2) (layer "F.Cu") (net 6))
 (segment (start 163.07 62.91) (end 160.41 62.91) (width 0.2) (layer "F.Cu") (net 6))
 (segment (start 143.6745 62.83) (end 143.515 62.83) (width 0.2) (layer "F.Cu") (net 6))
 (segment (start 160.41 62.91) (end 160.17 62.67) (width 0.2) (layer "F.Cu") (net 6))
 (segment (start 146.93 101.71) (end 163.79 101.71) (width 0.2) (layer "F.Cu") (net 6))
 (segment (start 146.225 91.31) (end 144.924 92.611) (width 0.2) (layer "F.Cu") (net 6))
 (segment (start 164.729 64.569) (end 163.07 62.91) (width 0.2) (layer "F.Cu") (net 6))
 (segment (start 143.7545 62.91) (end 143.6745 62.83) (width 0.2) (layer "F.Cu") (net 6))
 (segment (start 164.729 100.771) (end 164.729 100.68) (width 0.2) (layer "F.Cu") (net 6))
 (segment (start 164.729 100.68) (end 164.729 64.569) (width 0.2) (layer "F.Cu") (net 6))
 (segment (start 144.924 99.704) (end 146.93 101.71) (width 0.2) (layer "F.Cu") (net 6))
 (via (at 160.17 62.67) (size 0.6) (drill 0.3) (layers "F.Cu" "B.Cu") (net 6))
 (via (at 145.97 62.79) (size 0.6) (drill 0.3) (layers "F.Cu" "B.Cu") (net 6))
 (segment (start 146.09 62.67) (end 160.17 62.67) (width 0.2) (layer "B.Cu") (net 6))
 (segment (start 145.97 62.79) (end 146.09 62.67) (width 0.2) (layer "B.Cu") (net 6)))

